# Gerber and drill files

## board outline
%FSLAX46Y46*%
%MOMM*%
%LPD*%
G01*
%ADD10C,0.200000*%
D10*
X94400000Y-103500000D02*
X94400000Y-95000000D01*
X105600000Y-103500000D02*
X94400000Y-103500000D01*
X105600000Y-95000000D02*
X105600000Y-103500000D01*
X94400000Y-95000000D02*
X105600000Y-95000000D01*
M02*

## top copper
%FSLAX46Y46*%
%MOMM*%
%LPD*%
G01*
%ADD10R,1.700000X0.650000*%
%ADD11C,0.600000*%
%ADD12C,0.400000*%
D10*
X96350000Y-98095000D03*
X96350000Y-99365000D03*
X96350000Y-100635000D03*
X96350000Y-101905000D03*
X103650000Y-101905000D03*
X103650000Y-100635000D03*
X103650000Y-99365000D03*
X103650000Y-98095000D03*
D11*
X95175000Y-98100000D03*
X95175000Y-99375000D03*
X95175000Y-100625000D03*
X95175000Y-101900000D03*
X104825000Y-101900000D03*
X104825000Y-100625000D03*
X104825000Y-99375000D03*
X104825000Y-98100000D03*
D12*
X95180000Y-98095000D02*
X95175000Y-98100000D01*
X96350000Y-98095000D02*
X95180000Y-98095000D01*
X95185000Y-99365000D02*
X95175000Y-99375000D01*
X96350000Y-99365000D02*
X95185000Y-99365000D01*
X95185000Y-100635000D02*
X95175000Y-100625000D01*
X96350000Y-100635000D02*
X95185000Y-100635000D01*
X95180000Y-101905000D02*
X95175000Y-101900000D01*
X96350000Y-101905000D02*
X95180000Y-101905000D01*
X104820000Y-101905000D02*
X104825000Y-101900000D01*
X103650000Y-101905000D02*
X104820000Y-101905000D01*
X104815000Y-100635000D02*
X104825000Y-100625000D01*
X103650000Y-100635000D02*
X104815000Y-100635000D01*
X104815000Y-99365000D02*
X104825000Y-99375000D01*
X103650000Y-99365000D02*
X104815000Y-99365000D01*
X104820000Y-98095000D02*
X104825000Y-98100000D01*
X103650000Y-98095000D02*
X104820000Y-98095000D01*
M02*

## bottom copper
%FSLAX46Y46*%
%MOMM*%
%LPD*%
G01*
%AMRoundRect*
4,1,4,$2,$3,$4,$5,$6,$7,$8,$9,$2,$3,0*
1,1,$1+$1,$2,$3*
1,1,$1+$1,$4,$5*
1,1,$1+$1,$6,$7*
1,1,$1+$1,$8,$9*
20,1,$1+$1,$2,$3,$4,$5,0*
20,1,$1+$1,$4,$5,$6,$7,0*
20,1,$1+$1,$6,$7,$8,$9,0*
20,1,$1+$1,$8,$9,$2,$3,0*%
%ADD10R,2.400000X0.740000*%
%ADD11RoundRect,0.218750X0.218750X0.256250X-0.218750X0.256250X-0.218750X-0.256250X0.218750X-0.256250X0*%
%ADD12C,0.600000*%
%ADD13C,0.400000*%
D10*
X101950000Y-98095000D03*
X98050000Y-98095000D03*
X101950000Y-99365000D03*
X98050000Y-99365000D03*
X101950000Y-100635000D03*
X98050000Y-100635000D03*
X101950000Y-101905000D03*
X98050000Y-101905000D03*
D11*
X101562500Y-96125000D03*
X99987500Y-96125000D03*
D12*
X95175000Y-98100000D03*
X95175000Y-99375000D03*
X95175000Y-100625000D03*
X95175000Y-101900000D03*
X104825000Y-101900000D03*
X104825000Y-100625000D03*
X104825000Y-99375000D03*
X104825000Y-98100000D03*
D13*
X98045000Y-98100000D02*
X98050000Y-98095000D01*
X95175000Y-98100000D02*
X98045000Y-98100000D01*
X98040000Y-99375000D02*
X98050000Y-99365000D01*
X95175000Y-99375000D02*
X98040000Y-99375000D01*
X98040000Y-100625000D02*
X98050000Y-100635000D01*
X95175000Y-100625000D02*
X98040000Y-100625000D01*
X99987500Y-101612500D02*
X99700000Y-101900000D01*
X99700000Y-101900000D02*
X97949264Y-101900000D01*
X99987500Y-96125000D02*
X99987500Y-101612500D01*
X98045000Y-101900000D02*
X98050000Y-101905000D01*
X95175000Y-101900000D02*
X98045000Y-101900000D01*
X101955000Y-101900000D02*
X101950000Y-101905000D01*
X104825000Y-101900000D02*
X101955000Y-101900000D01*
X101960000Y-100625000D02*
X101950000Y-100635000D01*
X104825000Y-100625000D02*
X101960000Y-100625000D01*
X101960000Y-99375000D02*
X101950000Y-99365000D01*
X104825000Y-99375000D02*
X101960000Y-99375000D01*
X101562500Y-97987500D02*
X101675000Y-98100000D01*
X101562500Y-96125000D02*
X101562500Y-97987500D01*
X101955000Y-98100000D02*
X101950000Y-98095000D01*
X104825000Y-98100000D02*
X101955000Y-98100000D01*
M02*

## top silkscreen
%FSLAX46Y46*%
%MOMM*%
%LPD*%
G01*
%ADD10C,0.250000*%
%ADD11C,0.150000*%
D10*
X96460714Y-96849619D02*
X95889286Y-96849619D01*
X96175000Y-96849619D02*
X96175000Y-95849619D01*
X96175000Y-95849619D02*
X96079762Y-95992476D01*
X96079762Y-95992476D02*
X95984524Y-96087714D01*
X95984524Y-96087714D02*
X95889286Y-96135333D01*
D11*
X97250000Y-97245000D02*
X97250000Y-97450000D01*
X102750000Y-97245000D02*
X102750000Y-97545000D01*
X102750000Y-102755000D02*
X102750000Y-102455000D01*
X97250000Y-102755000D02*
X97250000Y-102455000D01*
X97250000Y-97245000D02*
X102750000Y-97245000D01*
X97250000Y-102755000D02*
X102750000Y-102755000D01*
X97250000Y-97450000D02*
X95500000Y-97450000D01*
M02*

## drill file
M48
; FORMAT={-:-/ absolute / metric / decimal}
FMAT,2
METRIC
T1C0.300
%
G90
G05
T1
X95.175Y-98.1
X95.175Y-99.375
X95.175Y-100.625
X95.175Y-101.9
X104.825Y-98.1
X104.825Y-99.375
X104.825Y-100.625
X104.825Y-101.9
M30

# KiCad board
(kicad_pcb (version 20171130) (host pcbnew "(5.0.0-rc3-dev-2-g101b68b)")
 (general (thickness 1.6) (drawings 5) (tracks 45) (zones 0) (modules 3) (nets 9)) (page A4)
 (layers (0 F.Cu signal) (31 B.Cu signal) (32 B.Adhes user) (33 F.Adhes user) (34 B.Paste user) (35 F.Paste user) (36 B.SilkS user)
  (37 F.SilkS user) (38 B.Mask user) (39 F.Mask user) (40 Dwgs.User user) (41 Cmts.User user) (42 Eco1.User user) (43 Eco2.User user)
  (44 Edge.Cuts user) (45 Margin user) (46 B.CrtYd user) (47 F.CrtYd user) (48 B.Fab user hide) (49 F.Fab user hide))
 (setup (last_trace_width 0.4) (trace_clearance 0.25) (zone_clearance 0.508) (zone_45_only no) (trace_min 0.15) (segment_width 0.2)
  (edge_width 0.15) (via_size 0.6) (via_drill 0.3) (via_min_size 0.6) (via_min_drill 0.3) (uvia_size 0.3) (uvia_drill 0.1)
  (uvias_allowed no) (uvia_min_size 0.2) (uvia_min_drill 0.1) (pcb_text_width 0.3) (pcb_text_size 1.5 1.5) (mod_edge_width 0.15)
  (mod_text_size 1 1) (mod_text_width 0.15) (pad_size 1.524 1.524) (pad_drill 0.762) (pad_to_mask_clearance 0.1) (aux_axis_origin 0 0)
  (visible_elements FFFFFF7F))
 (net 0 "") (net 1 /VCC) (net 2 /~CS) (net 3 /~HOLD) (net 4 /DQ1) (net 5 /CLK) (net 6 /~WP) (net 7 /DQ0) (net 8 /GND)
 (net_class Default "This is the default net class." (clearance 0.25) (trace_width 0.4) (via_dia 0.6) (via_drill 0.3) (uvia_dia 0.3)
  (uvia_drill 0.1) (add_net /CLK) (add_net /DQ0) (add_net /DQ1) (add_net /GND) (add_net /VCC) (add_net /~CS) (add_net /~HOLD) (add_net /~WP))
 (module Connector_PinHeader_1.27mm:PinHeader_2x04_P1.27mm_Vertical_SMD (layer B.Cu) (at 100 100 180)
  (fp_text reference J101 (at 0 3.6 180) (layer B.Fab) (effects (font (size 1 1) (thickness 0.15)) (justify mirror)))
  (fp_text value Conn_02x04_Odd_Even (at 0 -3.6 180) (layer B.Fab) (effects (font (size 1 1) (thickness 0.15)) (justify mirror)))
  (pad 1 smd rect (at -1.95 1.905 180) (size 2.4 0.74) (layers B.Cu B.Paste B.Mask) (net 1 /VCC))
  (pad 2 smd rect (at 1.95 1.905 180) (size 2.4 0.74) (layers B.Cu B.Paste B.Mask) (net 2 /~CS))
  (pad 3 smd rect (at -1.95 0.635 180) (size 2.4 0.74) (layers B.Cu B.Paste B.Mask) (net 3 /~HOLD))
  (pad 4 smd rect (at 1.95 0.635 180) (size 2.4 0.74) (layers B.Cu B.Paste B.Mask) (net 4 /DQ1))
  (pad 5 smd rect (at -1.95 -0.635 180) (size 2.4 0.74) (layers B.Cu B.Paste B.Mask) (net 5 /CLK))
  (pad 6 smd rect (at 1.95 -0.635 180) (size 2.4 0.74) (layers B.Cu B.Paste B.Mask) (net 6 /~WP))
  (pad 7 smd rect (at -1.95 -1.905 180) (size 2.4 0.74) (layers B.Cu B.Paste B.Mask) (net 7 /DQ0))
  (pad 8 smd rect (at 1.95 -1.905 180) (size 2.4 0.74) (layers B.Cu B.Paste B.Mask) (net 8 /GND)))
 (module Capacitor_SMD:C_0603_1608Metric (layer B.Cu) (at 100.775 96.125 180)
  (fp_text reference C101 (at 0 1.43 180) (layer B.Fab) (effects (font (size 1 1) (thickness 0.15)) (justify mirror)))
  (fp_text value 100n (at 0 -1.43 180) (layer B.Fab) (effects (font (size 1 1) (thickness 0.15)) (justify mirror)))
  (pad 1 smd roundrect (at -0.7875 0 180) (size 0.875 0.95) (layers B.Cu B.Paste B.Mask) (roundrect_rratio 0.25) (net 1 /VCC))
  (pad 2 smd roundrect (at 0.7875 0 180) (size 0.875 0.95) (layers B.Cu B.Paste B.Mask) (roundrect_rratio 0.25) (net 8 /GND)))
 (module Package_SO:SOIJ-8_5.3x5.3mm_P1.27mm (layer F.Cu) (at 100 100)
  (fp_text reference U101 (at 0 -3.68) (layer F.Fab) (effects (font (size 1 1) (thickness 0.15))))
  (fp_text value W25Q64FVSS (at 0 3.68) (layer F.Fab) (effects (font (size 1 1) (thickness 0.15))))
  (fp_line (start -2.75 -2.755) (end -2.75 -2.55) (layer F.SilkS) (width 0.15))
  (fp_line (start 2.75 -2.755) (end 2.75 -2.455) (layer F.SilkS) (width 0.15))
  (fp_line (start 2.75 2.755) (end 2.75 2.455) (layer F.SilkS) (width 0.15))
  (fp_line (start -2.75 2.755) (end -2.75 2.455) (layer F.SilkS) (width 0.15))
  (fp_line (start -2.75 -2.755) (end 2.75 -2.755) (layer F.SilkS) (width 0.15))
  (fp_line (start -2.75 2.755) (end 2.75 2.755) (layer F.SilkS) (width 0.15))
  (fp_line (start -2.75 -2.55) (end -4.5 -2.55) (layer F.SilkS) (width 0.15))
  (pad 1 smd rect (at -3.65 -1.905) (size 1.7 0.65) (layers F.Cu F.Paste F.Mask) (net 2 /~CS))
  (pad 2 smd rect (at -3.65 -0.635) (size 1.7 0.65) (layers F.Cu F.Paste F.Mask) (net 4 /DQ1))
  (pad 3 smd rect (at -3.65 0.635) (size 1.7 0.65) (layers F.Cu F.Paste F.Mask) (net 6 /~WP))
  (pad 4 smd rect (at -3.65 1.905) (size 1.7 0.65) (layers F.Cu F.Paste F.Mask) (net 8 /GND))
  (pad 5 smd rect (at 3.65 1.905) (size 1.7 0.65) (layers F.Cu F.Paste F.Mask) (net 7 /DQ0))
  (pad 6 smd rect (at 3.65 0.635) (size 1.7 0.65) (layers F.Cu F.Paste F.Mask) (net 5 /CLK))
  (pad 7 smd rect (at 3.65 -0.635) (size 1.7 0.65) (layers F.Cu F.Paste F.Mask) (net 3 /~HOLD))
  (pad 8 smd rect (at 3.65 -1.905) (size 1.7 0.65) (layers F.Cu F.Paste F.Mask) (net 1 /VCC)))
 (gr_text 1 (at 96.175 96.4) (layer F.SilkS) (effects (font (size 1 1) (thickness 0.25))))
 (gr_line (start 94.4 103.5) (end 94.4 95) (layer Edge.Cuts) (width 0.2))
 (gr_line (start 105.6 103.5) (end 94.4 103.5) (layer Edge.Cuts) (width 0.2))
 (gr_line (start 105.6 95) (end 105.6 103.5) (layer Edge.Cuts) (width 0.2))
 (gr_line (start 94.4 95) (end 105.6 95) (layer Edge.Cuts) (width 0.2))
 (via (at 95.175 98.1) (size 0.6) (drill 0.3) (layers F.Cu B.Cu) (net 2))
 (segment (start 95.18 98.095) (end 95.175 98.1) (width 0.4) (layer F.Cu) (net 2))
 (segment (start 96.35 98.095) (end 95.18 98.095) (width 0.4) (layer F.Cu) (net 2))
 (segment (start 98.045 98.1) (end 98.05 98.095) (width 0.4) (layer B.Cu) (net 2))
 (segment (start 95.175 98.1) (end 98.045 98.1) (width 0.4) (layer B.Cu) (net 2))
 (via (at 95.175 99.375) (size 0.6) (drill 0.3) (layers F.Cu B.Cu) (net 4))
 (segment (start 95.185 99.365) (end 95.175 99.375) (width 0.4) (layer F.Cu) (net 4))
 (segment (start 96.35 99.365) (end 95.185 99.365) (width 0.4) (layer F.Cu) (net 4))
 (segment (start 98.04 99.375) (end 98.05 99.365) (width 0.4) (layer B.Cu) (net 4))
 (segment (start 95.175 99.375) (end 98.04 99.375) (width 0.4) (layer B.Cu) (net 4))
 (via (at 95.175 100.625) (size 0.6) (drill 0.3) (layers F.Cu B.Cu) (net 6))
 (segment (start 95.185 100.635) (end 95.175 100.625) (width 0.4) (layer F.Cu) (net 6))
 (segment (start 96.35 100.635) (end 95.185 100.635) (width 0.4) (layer F.Cu) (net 6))
 (segment (start 98.04 100.625) (end 98.05 100.635) (width 0.4) (layer B.Cu) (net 6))
 (segment (start 95.175 100.625) (end 98.04 100.625) (width 0.4) (layer B.Cu) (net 6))
 (segment (start 99.9875 101.6125) (end 99.7 101.9) (width 0.4) (layer B.Cu) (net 8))
 (segment (start 99.7 101.9) (end 97.949264 101.9) (width 0.4) (layer B.Cu) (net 8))
 (segment (start 99.9875 96.125) (end 99.9875 101.6125) (width 0.4) (layer B.Cu) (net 8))
 (via (at 95.175 101.9) (size 0.6) (drill 0.3) (layers F.Cu B.Cu) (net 8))
 (segment (start 95.18 101.905) (end 95.175 101.9) (width 0.4) (layer F.Cu) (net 8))
 (segment (start 96.35 101.905) (end 95.18 101.905) (width 0.4) (layer F.Cu) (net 8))
 (segment (start 98.045 101.9) (end 98.05 101.905) (width 0.4) (layer B.Cu) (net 8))
 (segment (start 95.175 101.9) (end 98.045 101.9) (width 0.4) (layer B.Cu) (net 8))
 (via (at 104.825 101.9) (size 0.6) (drill 0.3) (layers F.Cu B.Cu) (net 7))
 (segment (start 104.82 101.905) (end 104.825 101.9) (width 0.4) (layer F.Cu) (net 7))
 (segment (start 103.65 101.905) (end 104.82 101.905) (width 0.4) (layer F.Cu) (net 7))
 (segment (start 101.955 101.9) (end 101.95 101.905) (width 0.4) (layer B.Cu) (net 7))
 (segment (start 104.825 101.9) (end 101.955 101.9) (width 0.4) (layer B.Cu) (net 7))
 (via (at 104.825 100.625) (size 0.6) (drill 0.3) (layers F.Cu B.Cu) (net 5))
 (segment (start 104.815 100.635) (end 104.825 100.625) (width 0.4) (layer F.Cu) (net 5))
 (segment (start 103.65 100.635) (end 104.815 100.635) (width 0.4) (layer F.Cu) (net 5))
 (segment (start 101.96 100.625) (end 101.95 100.635) (width 0.4) (layer B.Cu) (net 5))
 (segment (start 104.825 100.625) (end 101.96 100.625) (width 0.4) (layer B.Cu) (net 5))
 (via (at 104.825 99.375) (size 0.6) (drill 0.3) (layers F.Cu B.Cu) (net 3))
 (segment (start 104.815 99.365) (end 104.825 99.375) (width 0.4) (layer F.Cu) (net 3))
 (segment (start 103.65 99.365) (end 104.815 99.365) (width 0.4) (layer F.Cu) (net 3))
 (segment (start 101.96 99.375) (end 101.95 99.365) (width 0.4) (layer B.Cu) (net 3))
 (segment (start 104.825 99.375) (end 101.96 99.375) (width 0.4) (layer B.Cu) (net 3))
 (segment (start 101.5625 97.9875) (end 101.675 98.1) (width 0.4) (layer B.Cu) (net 1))
 (segment (start 101.5625 96.125) (end 101.5625 97.9875) (width 0.4) (layer B.Cu) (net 1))
 (via (at 104.825 98.1) (size 0.6) (drill 0.3) (layers F.Cu B.Cu) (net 1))
 (segment (start 104.82 98.095) (end 104.825 98.1) (width 0.4) (layer F.Cu) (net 1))
 (segment (start 103.65 98.095) (end 104.82 98.095) (width 0.4) (layer F.Cu) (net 1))
 (segment (start 101.955 98.1) (end 101.95 98.095) (width 0.4) (layer B.Cu) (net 1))
 (segment (start 104.825 98.1) (end 101.955 98.1) (width 0.4) (layer B.Cu) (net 1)))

